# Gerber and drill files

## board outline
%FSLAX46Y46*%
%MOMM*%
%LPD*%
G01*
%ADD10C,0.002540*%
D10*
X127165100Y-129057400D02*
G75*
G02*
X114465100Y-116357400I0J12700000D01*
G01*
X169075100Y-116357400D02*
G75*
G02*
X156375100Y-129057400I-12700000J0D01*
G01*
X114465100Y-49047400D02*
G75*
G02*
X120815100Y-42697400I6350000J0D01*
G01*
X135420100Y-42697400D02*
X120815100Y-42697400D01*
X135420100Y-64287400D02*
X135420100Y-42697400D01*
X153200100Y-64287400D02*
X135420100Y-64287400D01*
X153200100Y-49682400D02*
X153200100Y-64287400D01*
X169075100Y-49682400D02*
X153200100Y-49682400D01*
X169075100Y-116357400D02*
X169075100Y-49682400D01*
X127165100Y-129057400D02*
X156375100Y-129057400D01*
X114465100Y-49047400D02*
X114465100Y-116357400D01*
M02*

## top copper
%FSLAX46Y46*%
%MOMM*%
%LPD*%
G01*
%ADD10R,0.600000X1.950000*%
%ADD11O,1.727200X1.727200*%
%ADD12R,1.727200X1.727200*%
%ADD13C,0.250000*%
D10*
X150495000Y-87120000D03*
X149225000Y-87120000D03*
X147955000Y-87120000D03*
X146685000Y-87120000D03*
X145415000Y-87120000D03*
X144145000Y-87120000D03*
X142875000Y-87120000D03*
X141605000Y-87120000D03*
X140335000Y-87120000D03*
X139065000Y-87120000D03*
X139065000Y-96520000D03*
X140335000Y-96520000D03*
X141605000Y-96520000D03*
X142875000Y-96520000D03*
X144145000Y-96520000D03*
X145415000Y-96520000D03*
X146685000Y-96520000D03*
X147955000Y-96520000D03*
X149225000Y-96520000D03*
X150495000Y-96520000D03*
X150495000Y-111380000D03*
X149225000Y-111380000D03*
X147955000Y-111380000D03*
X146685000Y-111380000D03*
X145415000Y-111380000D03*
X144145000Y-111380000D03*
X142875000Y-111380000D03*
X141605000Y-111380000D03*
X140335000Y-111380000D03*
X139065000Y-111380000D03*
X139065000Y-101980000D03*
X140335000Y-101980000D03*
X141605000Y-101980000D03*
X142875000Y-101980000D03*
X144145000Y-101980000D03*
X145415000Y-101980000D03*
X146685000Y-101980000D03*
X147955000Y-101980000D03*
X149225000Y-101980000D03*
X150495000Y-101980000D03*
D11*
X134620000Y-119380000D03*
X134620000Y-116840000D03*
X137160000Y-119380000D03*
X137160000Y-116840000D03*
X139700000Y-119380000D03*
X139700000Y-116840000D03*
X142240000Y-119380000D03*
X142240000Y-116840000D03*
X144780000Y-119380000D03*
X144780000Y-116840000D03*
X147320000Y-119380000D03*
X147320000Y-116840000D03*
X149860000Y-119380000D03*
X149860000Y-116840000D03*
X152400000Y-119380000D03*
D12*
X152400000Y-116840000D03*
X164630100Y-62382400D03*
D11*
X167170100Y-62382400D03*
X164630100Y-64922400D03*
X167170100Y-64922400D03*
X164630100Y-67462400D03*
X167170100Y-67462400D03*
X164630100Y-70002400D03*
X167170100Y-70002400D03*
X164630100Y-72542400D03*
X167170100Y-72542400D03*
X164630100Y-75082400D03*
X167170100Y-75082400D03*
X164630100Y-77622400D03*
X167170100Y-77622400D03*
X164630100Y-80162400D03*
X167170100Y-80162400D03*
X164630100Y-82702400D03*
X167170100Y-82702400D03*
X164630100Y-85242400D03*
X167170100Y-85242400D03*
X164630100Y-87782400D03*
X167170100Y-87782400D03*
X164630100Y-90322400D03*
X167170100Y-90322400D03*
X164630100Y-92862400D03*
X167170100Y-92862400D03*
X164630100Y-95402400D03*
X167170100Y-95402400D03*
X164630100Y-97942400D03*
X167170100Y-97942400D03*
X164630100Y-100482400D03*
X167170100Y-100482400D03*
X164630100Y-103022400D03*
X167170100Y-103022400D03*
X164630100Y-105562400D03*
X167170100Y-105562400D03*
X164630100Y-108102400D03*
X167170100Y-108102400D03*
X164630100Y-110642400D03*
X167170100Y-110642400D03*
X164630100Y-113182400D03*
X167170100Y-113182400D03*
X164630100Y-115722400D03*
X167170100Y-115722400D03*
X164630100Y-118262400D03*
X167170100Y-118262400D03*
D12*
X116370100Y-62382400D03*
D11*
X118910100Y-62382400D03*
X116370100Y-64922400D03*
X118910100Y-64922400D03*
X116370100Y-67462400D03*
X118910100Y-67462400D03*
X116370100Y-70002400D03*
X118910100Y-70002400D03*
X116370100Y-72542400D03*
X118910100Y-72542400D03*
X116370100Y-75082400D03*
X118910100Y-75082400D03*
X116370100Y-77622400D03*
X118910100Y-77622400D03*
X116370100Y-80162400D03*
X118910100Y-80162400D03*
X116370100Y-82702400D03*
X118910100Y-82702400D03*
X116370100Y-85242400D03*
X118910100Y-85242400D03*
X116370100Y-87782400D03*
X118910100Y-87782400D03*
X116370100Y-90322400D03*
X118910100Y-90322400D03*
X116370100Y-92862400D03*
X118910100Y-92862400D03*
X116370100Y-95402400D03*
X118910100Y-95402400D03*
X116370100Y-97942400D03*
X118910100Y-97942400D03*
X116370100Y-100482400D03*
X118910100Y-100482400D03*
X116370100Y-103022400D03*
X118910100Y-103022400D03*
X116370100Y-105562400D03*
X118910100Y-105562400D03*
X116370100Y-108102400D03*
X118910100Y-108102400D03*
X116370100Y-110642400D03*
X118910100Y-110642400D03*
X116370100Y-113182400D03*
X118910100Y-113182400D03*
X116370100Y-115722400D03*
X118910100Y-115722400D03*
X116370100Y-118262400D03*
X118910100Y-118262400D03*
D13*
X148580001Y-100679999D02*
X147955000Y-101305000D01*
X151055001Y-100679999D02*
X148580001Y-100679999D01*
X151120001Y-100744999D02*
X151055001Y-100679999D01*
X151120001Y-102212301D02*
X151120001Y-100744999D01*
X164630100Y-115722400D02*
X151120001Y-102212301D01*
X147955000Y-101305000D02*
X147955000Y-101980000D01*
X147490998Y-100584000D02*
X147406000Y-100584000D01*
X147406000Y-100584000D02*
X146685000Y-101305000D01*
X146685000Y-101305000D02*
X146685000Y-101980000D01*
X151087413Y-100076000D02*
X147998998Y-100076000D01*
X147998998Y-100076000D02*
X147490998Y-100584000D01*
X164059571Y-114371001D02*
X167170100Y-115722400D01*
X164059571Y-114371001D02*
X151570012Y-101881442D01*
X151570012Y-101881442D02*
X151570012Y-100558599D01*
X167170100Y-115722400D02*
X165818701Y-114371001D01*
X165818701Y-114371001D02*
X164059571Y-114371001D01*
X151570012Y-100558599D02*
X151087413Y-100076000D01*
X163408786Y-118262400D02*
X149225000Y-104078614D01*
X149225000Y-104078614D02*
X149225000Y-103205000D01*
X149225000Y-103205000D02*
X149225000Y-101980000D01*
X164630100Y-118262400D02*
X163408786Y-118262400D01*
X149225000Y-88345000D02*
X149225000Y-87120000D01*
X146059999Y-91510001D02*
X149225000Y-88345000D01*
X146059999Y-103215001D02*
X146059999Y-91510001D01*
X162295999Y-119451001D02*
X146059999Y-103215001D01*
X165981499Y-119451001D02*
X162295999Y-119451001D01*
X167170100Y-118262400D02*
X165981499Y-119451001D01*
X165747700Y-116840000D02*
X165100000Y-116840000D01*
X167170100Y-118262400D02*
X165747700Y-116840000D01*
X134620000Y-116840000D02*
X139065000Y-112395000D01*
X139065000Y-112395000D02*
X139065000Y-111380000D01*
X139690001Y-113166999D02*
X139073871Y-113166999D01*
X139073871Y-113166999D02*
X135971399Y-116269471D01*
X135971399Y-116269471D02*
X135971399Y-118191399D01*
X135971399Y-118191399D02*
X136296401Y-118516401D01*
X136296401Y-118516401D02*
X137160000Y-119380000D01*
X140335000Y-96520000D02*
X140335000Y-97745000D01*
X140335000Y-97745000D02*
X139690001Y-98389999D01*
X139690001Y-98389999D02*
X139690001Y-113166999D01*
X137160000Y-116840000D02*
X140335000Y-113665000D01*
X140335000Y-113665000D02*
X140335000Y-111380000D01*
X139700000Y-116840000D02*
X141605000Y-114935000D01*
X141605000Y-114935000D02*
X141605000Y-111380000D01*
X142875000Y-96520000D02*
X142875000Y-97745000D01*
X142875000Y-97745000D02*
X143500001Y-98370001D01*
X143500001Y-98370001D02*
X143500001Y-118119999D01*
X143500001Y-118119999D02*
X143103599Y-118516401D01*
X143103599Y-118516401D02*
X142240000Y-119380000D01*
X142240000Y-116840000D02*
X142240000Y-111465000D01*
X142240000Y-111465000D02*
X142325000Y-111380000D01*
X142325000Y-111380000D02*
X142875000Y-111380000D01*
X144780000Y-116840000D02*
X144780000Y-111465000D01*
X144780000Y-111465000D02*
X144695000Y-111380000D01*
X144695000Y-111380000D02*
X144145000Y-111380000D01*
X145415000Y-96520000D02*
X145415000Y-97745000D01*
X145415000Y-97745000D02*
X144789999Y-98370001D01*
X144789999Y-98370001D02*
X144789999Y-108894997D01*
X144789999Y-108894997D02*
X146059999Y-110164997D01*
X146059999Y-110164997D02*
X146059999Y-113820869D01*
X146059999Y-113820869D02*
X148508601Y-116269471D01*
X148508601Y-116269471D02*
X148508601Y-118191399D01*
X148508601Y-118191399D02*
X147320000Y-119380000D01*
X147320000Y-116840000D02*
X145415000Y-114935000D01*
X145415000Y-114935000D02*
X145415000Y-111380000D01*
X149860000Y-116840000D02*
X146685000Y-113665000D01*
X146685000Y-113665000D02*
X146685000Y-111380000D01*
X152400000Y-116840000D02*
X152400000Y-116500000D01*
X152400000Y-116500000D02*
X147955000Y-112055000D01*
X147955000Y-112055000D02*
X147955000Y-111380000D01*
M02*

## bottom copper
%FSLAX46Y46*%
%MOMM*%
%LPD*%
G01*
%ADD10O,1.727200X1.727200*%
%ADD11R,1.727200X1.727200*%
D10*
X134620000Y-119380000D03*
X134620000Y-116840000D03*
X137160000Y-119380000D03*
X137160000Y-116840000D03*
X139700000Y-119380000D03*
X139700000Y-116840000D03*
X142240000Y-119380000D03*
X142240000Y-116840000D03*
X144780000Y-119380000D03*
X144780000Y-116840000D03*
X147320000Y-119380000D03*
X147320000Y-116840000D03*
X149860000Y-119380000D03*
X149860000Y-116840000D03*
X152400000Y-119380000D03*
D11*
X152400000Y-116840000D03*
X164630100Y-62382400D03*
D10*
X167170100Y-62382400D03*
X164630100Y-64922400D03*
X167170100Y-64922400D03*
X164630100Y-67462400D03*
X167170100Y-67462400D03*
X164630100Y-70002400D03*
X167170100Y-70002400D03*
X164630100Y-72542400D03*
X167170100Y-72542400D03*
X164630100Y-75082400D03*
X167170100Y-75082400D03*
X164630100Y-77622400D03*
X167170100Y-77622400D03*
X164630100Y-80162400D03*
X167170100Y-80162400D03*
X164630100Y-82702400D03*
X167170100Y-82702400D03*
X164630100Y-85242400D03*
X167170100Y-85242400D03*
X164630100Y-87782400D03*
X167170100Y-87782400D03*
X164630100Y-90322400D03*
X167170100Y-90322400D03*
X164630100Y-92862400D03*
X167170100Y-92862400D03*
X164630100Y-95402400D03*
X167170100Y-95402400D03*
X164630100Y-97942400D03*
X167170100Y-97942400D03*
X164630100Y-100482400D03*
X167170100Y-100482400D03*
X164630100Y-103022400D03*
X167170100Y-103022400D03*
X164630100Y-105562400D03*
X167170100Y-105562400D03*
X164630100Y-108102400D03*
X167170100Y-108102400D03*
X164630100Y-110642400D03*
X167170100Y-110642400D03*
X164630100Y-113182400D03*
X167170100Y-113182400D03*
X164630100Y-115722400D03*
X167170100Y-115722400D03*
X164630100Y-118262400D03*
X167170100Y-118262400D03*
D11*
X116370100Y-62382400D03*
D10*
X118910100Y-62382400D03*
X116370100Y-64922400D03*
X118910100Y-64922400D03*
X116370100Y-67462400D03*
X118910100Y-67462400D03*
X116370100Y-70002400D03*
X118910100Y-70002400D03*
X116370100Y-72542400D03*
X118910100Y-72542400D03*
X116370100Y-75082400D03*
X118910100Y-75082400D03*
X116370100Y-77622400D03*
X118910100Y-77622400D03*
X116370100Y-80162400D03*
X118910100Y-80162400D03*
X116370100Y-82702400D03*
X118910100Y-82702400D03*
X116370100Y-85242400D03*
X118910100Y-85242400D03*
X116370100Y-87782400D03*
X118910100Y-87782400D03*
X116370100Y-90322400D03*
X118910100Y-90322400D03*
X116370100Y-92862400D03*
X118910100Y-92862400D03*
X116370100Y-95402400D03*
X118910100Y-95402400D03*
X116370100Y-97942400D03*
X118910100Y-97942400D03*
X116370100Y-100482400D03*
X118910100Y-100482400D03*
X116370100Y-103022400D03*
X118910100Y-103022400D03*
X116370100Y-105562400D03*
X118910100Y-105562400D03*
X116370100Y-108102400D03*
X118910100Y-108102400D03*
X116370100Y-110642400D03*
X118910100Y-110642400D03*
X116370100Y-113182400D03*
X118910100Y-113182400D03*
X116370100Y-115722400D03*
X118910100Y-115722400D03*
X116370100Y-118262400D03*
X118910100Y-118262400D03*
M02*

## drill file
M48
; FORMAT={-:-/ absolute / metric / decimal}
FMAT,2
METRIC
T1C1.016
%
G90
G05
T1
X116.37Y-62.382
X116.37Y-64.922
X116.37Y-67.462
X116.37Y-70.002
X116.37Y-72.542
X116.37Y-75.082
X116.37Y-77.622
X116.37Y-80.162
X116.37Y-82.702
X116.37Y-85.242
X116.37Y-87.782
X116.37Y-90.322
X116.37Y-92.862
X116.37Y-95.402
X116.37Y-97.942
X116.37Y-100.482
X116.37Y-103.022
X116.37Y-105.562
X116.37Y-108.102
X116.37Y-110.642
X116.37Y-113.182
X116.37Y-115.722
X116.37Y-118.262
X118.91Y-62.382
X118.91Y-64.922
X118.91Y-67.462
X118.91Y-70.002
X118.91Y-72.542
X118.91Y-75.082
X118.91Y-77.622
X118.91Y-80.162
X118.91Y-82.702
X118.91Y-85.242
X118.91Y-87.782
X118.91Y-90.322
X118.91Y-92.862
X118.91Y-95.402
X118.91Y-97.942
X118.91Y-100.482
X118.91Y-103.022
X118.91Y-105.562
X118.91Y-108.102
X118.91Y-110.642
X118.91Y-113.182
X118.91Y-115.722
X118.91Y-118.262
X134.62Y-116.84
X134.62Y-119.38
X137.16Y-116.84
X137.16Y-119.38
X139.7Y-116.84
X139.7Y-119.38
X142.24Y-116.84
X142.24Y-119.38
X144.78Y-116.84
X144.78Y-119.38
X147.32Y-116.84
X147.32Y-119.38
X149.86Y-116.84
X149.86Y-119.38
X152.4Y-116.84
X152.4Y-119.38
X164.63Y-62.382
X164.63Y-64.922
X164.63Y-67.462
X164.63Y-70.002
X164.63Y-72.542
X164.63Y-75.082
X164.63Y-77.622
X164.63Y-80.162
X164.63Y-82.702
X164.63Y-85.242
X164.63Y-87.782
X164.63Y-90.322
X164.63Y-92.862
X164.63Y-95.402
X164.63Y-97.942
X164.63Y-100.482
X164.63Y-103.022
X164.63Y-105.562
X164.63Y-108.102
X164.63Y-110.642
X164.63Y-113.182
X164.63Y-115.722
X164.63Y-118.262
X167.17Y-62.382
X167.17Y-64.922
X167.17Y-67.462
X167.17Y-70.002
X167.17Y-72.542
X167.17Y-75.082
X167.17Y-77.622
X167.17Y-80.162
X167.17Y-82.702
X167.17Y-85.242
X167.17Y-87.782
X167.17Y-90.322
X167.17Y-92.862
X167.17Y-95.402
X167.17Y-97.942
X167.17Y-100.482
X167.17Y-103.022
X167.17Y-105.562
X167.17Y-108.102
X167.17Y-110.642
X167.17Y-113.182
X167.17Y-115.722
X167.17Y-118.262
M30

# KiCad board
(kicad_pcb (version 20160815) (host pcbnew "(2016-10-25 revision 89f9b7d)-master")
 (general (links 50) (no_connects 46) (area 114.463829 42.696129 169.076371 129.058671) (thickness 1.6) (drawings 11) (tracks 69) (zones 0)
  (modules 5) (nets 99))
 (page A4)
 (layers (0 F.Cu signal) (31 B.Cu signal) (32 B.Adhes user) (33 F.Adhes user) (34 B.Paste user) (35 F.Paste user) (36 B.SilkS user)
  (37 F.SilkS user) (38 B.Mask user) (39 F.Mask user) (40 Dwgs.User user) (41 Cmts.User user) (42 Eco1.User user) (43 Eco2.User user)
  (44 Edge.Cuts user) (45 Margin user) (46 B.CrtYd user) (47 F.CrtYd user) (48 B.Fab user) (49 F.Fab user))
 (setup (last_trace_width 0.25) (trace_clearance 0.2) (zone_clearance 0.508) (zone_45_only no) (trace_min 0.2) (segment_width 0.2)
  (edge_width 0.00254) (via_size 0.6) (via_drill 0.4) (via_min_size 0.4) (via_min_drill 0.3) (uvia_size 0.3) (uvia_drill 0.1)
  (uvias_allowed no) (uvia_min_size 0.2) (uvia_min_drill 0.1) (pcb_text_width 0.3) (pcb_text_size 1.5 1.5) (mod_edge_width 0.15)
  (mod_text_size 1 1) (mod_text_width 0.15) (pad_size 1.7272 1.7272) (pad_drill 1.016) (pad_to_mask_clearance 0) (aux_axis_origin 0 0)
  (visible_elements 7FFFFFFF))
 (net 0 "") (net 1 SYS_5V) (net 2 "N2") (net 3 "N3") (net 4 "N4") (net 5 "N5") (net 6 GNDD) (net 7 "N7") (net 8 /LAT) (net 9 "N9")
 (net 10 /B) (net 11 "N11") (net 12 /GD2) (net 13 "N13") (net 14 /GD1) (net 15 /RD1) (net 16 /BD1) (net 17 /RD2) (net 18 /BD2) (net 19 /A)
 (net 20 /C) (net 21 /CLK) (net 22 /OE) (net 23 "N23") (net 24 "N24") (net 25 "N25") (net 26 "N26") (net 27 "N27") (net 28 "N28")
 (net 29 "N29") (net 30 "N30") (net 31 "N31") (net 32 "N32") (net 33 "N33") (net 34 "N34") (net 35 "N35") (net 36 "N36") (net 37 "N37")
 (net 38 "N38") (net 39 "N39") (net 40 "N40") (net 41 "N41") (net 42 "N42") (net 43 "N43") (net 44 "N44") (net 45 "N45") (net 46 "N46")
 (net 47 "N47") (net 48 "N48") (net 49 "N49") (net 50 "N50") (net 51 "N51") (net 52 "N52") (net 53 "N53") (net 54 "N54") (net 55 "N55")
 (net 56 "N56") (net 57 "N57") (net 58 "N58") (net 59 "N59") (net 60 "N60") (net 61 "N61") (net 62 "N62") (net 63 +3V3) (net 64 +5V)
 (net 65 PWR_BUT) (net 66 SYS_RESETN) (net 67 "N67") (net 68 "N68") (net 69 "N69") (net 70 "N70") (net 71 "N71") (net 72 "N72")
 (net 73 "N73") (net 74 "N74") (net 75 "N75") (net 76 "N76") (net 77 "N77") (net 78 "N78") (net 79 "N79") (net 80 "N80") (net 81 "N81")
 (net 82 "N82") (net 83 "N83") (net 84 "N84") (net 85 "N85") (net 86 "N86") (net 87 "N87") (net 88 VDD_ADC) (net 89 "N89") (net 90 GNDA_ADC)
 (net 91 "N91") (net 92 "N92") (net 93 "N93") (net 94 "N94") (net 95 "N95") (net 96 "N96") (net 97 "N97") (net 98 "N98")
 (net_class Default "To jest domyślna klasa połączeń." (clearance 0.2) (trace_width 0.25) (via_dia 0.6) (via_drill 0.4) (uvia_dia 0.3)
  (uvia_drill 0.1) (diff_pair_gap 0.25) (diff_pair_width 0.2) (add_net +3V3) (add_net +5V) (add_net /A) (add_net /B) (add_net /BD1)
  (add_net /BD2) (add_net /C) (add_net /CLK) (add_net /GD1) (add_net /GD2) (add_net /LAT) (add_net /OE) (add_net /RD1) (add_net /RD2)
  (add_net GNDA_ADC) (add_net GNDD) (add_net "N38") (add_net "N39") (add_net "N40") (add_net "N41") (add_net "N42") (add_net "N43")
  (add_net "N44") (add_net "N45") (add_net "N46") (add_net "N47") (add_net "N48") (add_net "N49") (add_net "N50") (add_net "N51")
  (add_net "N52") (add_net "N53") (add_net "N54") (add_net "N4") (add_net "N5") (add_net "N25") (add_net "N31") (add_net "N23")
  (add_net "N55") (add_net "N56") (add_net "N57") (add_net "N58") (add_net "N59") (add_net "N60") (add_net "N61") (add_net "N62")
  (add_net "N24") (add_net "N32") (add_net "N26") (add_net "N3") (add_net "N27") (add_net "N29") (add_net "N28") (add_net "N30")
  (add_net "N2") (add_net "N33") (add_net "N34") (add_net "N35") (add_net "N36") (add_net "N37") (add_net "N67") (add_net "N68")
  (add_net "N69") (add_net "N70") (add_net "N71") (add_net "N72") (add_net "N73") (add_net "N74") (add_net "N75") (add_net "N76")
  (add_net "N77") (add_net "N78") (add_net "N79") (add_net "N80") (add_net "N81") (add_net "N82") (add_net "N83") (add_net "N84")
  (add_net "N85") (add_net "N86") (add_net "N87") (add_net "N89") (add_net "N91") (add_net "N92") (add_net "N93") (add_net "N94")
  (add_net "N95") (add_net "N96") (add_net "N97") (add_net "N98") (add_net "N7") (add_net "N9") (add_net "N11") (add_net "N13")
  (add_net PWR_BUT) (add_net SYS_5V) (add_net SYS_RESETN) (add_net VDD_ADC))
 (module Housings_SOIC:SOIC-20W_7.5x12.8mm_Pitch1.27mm (layer F.Cu) (at 144.78 91.82 270)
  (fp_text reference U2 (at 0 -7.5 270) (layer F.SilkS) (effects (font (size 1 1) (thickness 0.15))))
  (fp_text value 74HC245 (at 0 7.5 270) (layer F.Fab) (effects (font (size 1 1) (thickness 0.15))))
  (pad 1 smd rect (at -4.7 -5.715 270) (size 1.95 0.6) (layers F.Cu F.Paste F.Mask) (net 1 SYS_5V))
  (pad 2 smd rect (at -4.7 -4.445 270) (size 1.95 0.6) (layers F.Cu F.Paste F.Mask) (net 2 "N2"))
  (pad 3 smd rect (at -4.7 -3.175 270) (size 1.95 0.6) (layers F.Cu F.Paste F.Mask) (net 1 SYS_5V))
  (pad 4 smd rect (at -4.7 -1.905 270) (size 1.95 0.6) (layers F.Cu F.Paste F.Mask) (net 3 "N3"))
  (pad 5 smd rect (at -4.7 -0.635 270) (size 1.95 0.6) (layers F.Cu F.Paste F.Mask) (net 1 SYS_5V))
  (pad 6 smd rect (at -4.7 0.635 270) (size 1.95 0.6) (layers F.Cu F.Paste F.Mask) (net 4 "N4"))
  (pad 7 smd rect (at -4.7 1.905 270) (size 1.95 0.6) (layers F.Cu F.Paste F.Mask) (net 1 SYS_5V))
  (pad 8 smd rect (at -4.7 3.175 270) (size 1.95 0.6) (layers F.Cu F.Paste F.Mask) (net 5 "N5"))
  (pad 9 smd rect (at -4.7 4.445 270) (size 1.95 0.6) (layers F.Cu F.Paste F.Mask) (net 1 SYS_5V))
  (pad 10 smd rect (at -4.7 5.715 270) (size 1.95 0.6) (layers F.Cu F.Paste F.Mask) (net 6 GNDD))
  (pad 11 smd rect (at 4.7 5.715 270) (size 1.95 0.6) (layers F.Cu F.Paste F.Mask) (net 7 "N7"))
  (pad 12 smd rect (at 4.7 4.445 270) (size 1.95 0.6) (layers F.Cu F.Paste F.Mask) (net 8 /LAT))
  (pad 13 smd rect (at 4.7 3.175 270) (size 1.95 0.6) (layers F.Cu F.Paste F.Mask) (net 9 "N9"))
  (pad 14 smd rect (at 4.7 1.905 270) (size 1.95 0.6) (layers F.Cu F.Paste F.Mask) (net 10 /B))
  (pad 15 smd rect (at 4.7 0.635 270) (size 1.95 0.6) (layers F.Cu F.Paste F.Mask) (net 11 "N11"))
  (pad 16 smd rect (at 4.7 -0.635 270) (size 1.95 0.6) (layers F.Cu F.Paste F.Mask) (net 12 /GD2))
  (pad 17 smd rect (at 4.7 -1.905 270) (size 1.95 0.6) (layers F.Cu F.Paste F.Mask) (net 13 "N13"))
  (pad 18 smd rect (at 4.7 -3.175 270) (size 1.95 0.6) (layers F.Cu F.Paste F.Mask) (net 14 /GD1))
  (pad 19 smd rect (at 4.7 -4.445 270) (size 1.95 0.6) (layers F.Cu F.Paste F.Mask) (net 6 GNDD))
  (pad 20 smd rect (at 4.7 -5.715 270) (size 1.95 0.6) (layers F.Cu F.Paste F.Mask) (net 1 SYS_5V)))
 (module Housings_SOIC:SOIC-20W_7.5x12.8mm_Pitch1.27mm (layer F.Cu) (at 144.78 106.68 270)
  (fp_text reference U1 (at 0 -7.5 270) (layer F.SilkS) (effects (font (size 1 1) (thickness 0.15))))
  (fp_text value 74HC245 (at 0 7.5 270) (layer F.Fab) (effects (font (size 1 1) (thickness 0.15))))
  (pad 20 smd rect (at 4.7 -5.715 270) (size 1.95 0.6) (layers F.Cu F.Paste F.Mask) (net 1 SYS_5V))
  (pad 19 smd rect (at 4.7 -4.445 270) (size 1.95 0.6) (layers F.Cu F.Paste F.Mask) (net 6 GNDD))
  (pad 18 smd rect (at 4.7 -3.175 270) (size 1.95 0.6) (layers F.Cu F.Paste F.Mask) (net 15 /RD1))
  (pad 17 smd rect (at 4.7 -1.905 270) (size 1.95 0.6) (layers F.Cu F.Paste F.Mask) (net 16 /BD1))
  (pad 16 smd rect (at 4.7 -0.635 270) (size 1.95 0.6) (layers F.Cu F.Paste F.Mask) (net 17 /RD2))
  (pad 15 smd rect (at 4.7 0.635 270) (size 1.95 0.6) (layers F.Cu F.Paste F.Mask) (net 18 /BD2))
  (pad 14 smd rect (at 4.7 1.905 270) (size 1.95 0.6) (layers F.Cu F.Paste F.Mask) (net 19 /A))
  (pad 13 smd rect (at 4.7 3.175 270) (size 1.95 0.6) (layers F.Cu F.Paste F.Mask) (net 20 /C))
  (pad 12 smd rect (at 4.7 4.445 270) (size 1.95 0.6) (layers F.Cu F.Paste F.Mask) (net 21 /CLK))
  (pad 11 smd rect (at 4.7 5.715 270) (size 1.95 0.6) (layers F.Cu F.Paste F.Mask) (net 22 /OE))
  (pad 10 smd rect (at -4.7 5.715 270) (size 1.95 0.6) (layers F.Cu F.Paste F.Mask) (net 6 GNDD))
  (pad 9 smd rect (at -4.7 4.445 270) (size 1.95 0.6) (layers F.Cu F.Paste F.Mask) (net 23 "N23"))
  (pad 8 smd rect (at -4.7 3.175 270) (size 1.95 0.6) (layers F.Cu F.Paste F.Mask) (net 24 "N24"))
  (pad 7 smd rect (at -4.7 1.905 270) (size 1.95 0.6) (layers F.Cu F.Paste F.Mask) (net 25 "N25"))
  (pad 6 smd rect (at -4.7 0.635 270) (size 1.95 0.6) (layers F.Cu F.Paste F.Mask) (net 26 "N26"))
  (pad 5 smd rect (at -4.7 -0.635 270) (size 1.95 0.6) (layers F.Cu F.Paste F.Mask) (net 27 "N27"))
  (pad 4 smd rect (at -4.7 -1.905 270) (size 1.95 0.6) (layers F.Cu F.Paste F.Mask) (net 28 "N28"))
  (pad 3 smd rect (at -4.7 -3.175 270) (size 1.95 0.6) (layers F.Cu F.Paste F.Mask) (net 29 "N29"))
  (pad 2 smd rect (at -4.7 -4.445 270) (size 1.95 0.6) (layers F.Cu F.Paste F.Mask) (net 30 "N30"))
  (pad 1 smd rect (at -4.7 -5.715 270) (size 1.95 0.6) (layers F.Cu F.Paste F.Mask) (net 1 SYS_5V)))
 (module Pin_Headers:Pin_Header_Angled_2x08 (layer F.Cu) (at 152.4 116.84 270)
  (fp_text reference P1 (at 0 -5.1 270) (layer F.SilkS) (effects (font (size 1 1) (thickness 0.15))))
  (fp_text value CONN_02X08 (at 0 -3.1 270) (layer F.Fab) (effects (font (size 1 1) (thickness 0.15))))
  (pad 16 thru_hole oval (at 2.54 17.78 270) (size 1.7272 1.7272) (drill 1.016) (layers *.Cu *.Mask F.SilkS) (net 6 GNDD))
  (pad 15 thru_hole oval (at 0 17.78 270) (size 1.7272 1.7272) (drill 1.016) (layers *.Cu *.Mask F.SilkS) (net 22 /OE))
  (pad 14 thru_hole oval (at 2.54 15.24 270) (size 1.7272 1.7272) (drill 1.016) (layers *.Cu *.Mask F.SilkS) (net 8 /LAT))
  (pad 13 thru_hole oval (at 0 15.24 270) (size 1.7272 1.7272) (drill 1.016) (layers *.Cu *.Mask F.SilkS) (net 21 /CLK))
  (pad 12 thru_hole oval (at 2.54 12.7 270) (size 1.7272 1.7272) (drill 1.016) (layers *.Cu *.Mask F.SilkS) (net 6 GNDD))
  (pad 11 thru_hole oval (at 0 12.7 270) (size 1.7272 1.7272) (drill 1.016) (layers *.Cu *.Mask F.SilkS) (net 20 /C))
  (pad 10 thru_hole oval (at 2.54 10.16 270) (size 1.7272 1.7272) (drill 1.016) (layers *.Cu *.Mask F.SilkS) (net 10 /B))
  (pad 9 thru_hole oval (at 0 10.16 270) (size 1.7272 1.7272) (drill 1.016) (layers *.Cu *.Mask F.SilkS) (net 19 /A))
  (pad 8 thru_hole oval (at 2.54 7.62 270) (size 1.7272 1.7272) (drill 1.016) (layers *.Cu *.Mask F.SilkS) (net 6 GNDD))
  (pad 7 thru_hole oval (at 0 7.62 270) (size 1.7272 1.7272) (drill 1.016) (layers *.Cu *.Mask F.SilkS) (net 18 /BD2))
  (pad 6 thru_hole oval (at 2.54 5.08 270) (size 1.7272 1.7272) (drill 1.016) (layers *.Cu *.Mask F.SilkS) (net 12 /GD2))
  (pad 5 thru_hole oval (at 0 5.08 270) (size 1.7272 1.7272) (drill 1.016) (layers *.Cu *.Mask F.SilkS) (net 17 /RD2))
  (pad 4 thru_hole oval (at 2.54 2.54 270) (size 1.7272 1.7272) (drill 1.016) (layers *.Cu *.Mask F.SilkS) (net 6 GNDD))
  (pad 3 thru_hole oval (at 0 2.54 270) (size 1.7272 1.7272) (drill 1.016) (layers *.Cu *.Mask F.SilkS) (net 16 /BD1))
  (pad 2 thru_hole oval (at 2.54 0 270) (size 1.7272 1.7272) (drill 1.016) (layers *.Cu *.Mask F.SilkS) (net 14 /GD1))
  (pad 1 thru_hole rect (at 0 0 270) (size 1.7272 1.7272) (drill 1.016) (layers *.Cu *.Mask F.SilkS) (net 15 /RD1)))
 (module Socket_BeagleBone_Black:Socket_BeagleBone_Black (layer F.Cu) (at 164.6301 62.3824)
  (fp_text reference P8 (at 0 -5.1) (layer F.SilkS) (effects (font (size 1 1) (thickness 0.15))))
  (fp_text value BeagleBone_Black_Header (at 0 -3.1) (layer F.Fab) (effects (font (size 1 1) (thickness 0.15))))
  (pad 1 thru_hole rect (at 0 0) (size 1.7272 1.7272) (drill 1.016) (layers *.Cu *.Mask F.SilkS) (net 6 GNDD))
  (pad 2 thru_hole oval (at 2.54 0) (size 1.7272 1.7272) (drill 1.016) (layers *.Cu *.Mask F.SilkS) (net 6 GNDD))
  (pad 3 thru_hole oval (at 0 2.54) (size 1.7272 1.7272) (drill 1.016) (layers *.Cu *.Mask F.SilkS) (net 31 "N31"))
  (pad 4 thru_hole oval (at 2.54 2.54) (size 1.7272 1.7272) (drill 1.016) (layers *.Cu *.Mask F.SilkS) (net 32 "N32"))
  (pad 5 thru_hole oval (at 0 5.08) (size 1.7272 1.7272) (drill 1.016) (layers *.Cu *.Mask F.SilkS) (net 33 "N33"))
  (pad 6 thru_hole oval (at 2.54 5.08) (size 1.7272 1.7272) (drill 1.016) (layers *.Cu *.Mask F.SilkS) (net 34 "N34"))
  (pad 7 thru_hole oval (at 0 7.62) (size 1.7272 1.7272) (drill 1.016) (layers *.Cu *.Mask F.SilkS) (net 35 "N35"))
  (pad 8 thru_hole oval (at 2.54 7.62) (size 1.7272 1.7272) (drill 1.016) (layers *.Cu *.Mask F.SilkS) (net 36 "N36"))
  (pad 9 thru_hole oval (at 0 10.16) (size 1.7272 1.7272) (drill 1.016) (layers *.Cu *.Mask F.SilkS) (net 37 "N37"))
  (pad 10 thru_hole oval (at 2.54 10.16) (size 1.7272 1.7272) (drill 1.016) (layers *.Cu *.Mask F.SilkS) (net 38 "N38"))
  (pad 11 thru_hole oval (at 0 12.7) (size 1.7272 1.7272) (drill 1.016) (layers *.Cu *.Mask F.SilkS) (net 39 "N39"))
  (pad 12 thru_hole oval (at 2.54 12.7) (size 1.7272 1.7272) (drill 1.016) (layers *.Cu *.Mask F.SilkS) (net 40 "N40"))
  (pad 13 thru_hole oval (at 0 15.24) (size 1.7272 1.7272) (drill 1.016) (layers *.Cu *.Mask F.SilkS) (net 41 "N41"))
  (pad 14 thru_hole oval (at 2.54 15.24) (size 1.7272 1.7272) (drill 1.016) (layers *.Cu *.Mask F.SilkS) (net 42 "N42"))
  (pad 15 thru_hole oval (at 0 17.78) (size 1.7272 1.7272) (drill 1.016) (layers *.Cu *.Mask F.SilkS) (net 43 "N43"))
  (pad 16 thru_hole oval (at 2.54 17.78) (size 1.7272 1.7272) (drill 1.016) (layers *.Cu *.Mask F.SilkS) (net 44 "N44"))
  (pad 17 thru_hole oval (at 0 20.32) (size 1.7272 1.7272) (drill 1.016) (layers *.Cu *.Mask F.SilkS) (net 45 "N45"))
  (pad 18 thru_hole oval (at 2.54 20.32) (size 1.7272 1.7272) (drill 1.016) (layers *.Cu *.Mask F.SilkS) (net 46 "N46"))
  (pad 19 thru_hole oval (at 0 22.86) (size 1.7272 1.7272) (drill 1.016) (layers *.Cu *.Mask F.SilkS) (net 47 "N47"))
  (pad 20 thru_hole oval (at 2.54 22.86) (size 1.7272 1.7272) (drill 1.016) (layers *.Cu *.Mask F.SilkS) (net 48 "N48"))
  (pad 21 thru_hole oval (at 0 25.4) (size 1.7272 1.7272) (drill 1.016) (layers *.Cu *.Mask F.SilkS) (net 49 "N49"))
  (pad 22 thru_hole oval (at 2.54 25.4) (size 1.7272 1.7272) (drill 1.016) (layers *.Cu *.Mask F.SilkS) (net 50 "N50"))
  (pad 23 thru_hole oval (at 0 27.94) (size 1.7272 1.7272) (drill 1.016) (layers *.Cu *.Mask F.SilkS) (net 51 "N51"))
  (pad 24 thru_hole oval (at 2.54 27.94) (size 1.7272 1.7272) (drill 1.016) (layers *.Cu *.Mask F.SilkS) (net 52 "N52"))
  (pad 25 thru_hole oval (at 0 30.48) (size 1.7272 1.7272) (drill 1.016) (layers *.Cu *.Mask F.SilkS) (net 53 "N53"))
  (pad 26 thru_hole oval (at 2.54 30.48) (size 1.7272 1.7272) (drill 1.016) (layers *.Cu *.Mask F.SilkS) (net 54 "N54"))
  (pad 27 thru_hole oval (at 0 33.02) (size 1.7272 1.7272) (drill 1.016) (layers *.Cu *.Mask F.SilkS) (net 4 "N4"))
  (pad 28 thru_hole oval (at 2.54 33.02) (size 1.7272 1.7272) (drill 1.016) (layers *.Cu *.Mask F.SilkS) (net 5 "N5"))
  (pad 29 thru_hole oval (at 0 35.56) (size 1.7272 1.7272) (drill 1.016) (layers *.Cu *.Mask F.SilkS) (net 25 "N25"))
  (pad 30 thru_hole oval (at 2.54 35.56) (size 1.7272 1.7272) (drill 1.016) (layers *.Cu *.Mask F.SilkS) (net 23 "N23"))
  (pad 31 thru_hole oval (at 0 38.1) (size 1.7272 1.7272) (drill 1.016) (layers *.Cu *.Mask F.SilkS) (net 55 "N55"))
  (pad 32 thru_hole oval (at 2.54 38.1) (size 1.7272 1.7272) (drill 1.016) (layers *.Cu *.Mask F.SilkS) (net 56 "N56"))
  (pad 33 thru_hole oval (at 0 40.64) (size 1.7272 1.7272) (drill 1.016) (layers *.Cu *.Mask F.SilkS) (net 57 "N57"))
  (pad 34 thru_hole oval (at 2.54 40.64) (size 1.7272 1.7272) (drill 1.016) (layers *.Cu *.Mask F.SilkS) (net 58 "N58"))
  (pad 35 thru_hole oval (at 0 43.18) (size 1.7272 1.7272) (drill 1.016) (layers *.Cu *.Mask F.SilkS) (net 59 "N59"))
  (pad 36 thru_hole oval (at 2.54 43.18) (size 1.7272 1.7272) (drill 1.016) (layers *.Cu *.Mask F.SilkS) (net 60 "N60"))
  (pad 37 thru_hole oval (at 0 45.72) (size 1.7272 1.7272) (drill 1.016) (layers *.Cu *.Mask F.SilkS) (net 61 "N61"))
  (pad 38 thru_hole oval (at 2.54 45.72) (size 1.7272 1.7272) (drill 1.016) (layers *.Cu *.Mask F.SilkS) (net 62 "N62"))
  (pad 39 thru_hole oval (at 0 48.26) (size 1.7272 1.7272) (drill 1.016) (layers *.Cu *.Mask F.SilkS) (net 24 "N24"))
  (pad 40 thru_hole oval (at 2.54 48.26) (size 1.7272 1.7272) (drill 1.016) (layers *.Cu *.Mask F.SilkS) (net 26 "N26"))
  (pad 41 thru_hole oval (at 0 50.8) (size 1.7272 1.7272) (drill 1.016) (layers *.Cu *.Mask F.SilkS) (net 3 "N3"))
  (pad 42 thru_hole oval (at 2.54 50.8) (size 1.7272 1.7272) (drill 1.016) (layers *.Cu *.Mask F.SilkS) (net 27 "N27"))
  (pad 43 thru_hole oval (at 0 53.34) (size 1.7272 1.7272) (drill 1.016) (layers *.Cu *.Mask F.SilkS) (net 29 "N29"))
  (pad 44 thru_hole oval (at 2.54 53.34) (size 1.7272 1.7272) (drill 1.016) (layers *.Cu *.Mask F.SilkS) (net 28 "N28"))
  (pad 45 thru_hole oval (at 0 55.88) (size 1.7272 1.7272) (drill 1.016) (layers *.Cu *.Mask F.SilkS) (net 30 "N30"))
  (pad 46 thru_hole oval (at 2.54 55.88) (size 1.7272 1.7272) (drill 1.016) (layers *.Cu *.Mask F.SilkS) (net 2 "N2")))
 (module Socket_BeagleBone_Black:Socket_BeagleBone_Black (layer F.Cu) (at 116.3701 62.3824)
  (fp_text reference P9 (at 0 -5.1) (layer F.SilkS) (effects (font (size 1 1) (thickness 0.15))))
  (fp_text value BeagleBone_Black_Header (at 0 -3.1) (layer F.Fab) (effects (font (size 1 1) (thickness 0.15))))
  (pad 1 thru_hole rect (at 0 0) (size 1.7272 1.7272) (drill 1.016) (layers *.Cu *.Mask F.SilkS) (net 6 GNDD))
  (pad 2 thru_hole oval (at 2.54 0) (size 1.7272 1.7272) (drill 1.016) (layers *.Cu *.Mask F.SilkS) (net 6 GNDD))
  (pad 3 thru_hole oval (at 0 2.54) (size 1.7272 1.7272) (drill 1.016) (layers *.Cu *.Mask F.SilkS) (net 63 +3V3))
  (pad 4 thru_hole oval (at 2.54 2.54) (size 1.7272 1.7272) (drill 1.016) (layers *.Cu *.Mask F.SilkS) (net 63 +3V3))
  (pad 5 thru_hole oval (at 0 5.08) (size 1.7272 1.7272) (drill 1.016) (layers *.Cu *.Mask F.SilkS) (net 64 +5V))
  (pad 6 thru_hole oval (at 2.54 5.08) (size 1.7272 1.7272) (drill 1.016) (layers *.Cu *.Mask F.SilkS) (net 64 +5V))
  (pad 7 thru_hole oval (at 0 7.62) (size 1.7272 1.7272) (drill 1.016) (layers *.Cu *.Mask F.SilkS) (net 1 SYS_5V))
  (pad 8 thru_hole oval (at 2.54 7.62) (size 1.7272 1.7272) (drill 1.016) (layers *.Cu *.Mask F.SilkS) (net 1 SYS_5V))
  (pad 9 thru_hole oval (at 0 10.16) (size 1.7272 1.7272) (drill 1.016) (layers *.Cu *.Mask F.SilkS) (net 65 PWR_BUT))
  (pad 10 thru_hole oval (at 2.54 10.16) (size 1.7272 1.7272) (drill 1.016) (layers *.Cu *.Mask F.SilkS) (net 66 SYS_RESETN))
  (pad 11 thru_hole oval (at 0 12.7) (size 1.7272 1.7272) (drill 1.016) (layers *.Cu *.Mask F.SilkS) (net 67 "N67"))
  (pad 12 thru_hole oval (at 2.54 12.7) (size 1.7272 1.7272) (drill 1.016) (layers *.Cu *.Mask F.SilkS) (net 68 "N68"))
  (pad 13 thru_hole oval (at 0 15.24) (size 1.7272 1.7272) (drill 1.016) (layers *.Cu *.Mask F.SilkS) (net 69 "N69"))
  (pad 14 thru_hole oval (at 2.54 15.24) (size 1.7272 1.7272) (drill 1.016) (layers *.Cu *.Mask F.SilkS) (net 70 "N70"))
  (pad 15 thru_hole oval (at 0 17.78) (size 1.7272 1.7272) (drill 1.016) (layers *.Cu *.Mask F.SilkS) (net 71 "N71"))
  (pad 16 thru_hole oval (at 2.54 17.78) (size 1.7272 1.7272) (drill 1.016) (layers *.Cu *.Mask F.SilkS) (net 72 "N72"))
  (pad 17 thru_hole oval (at 0 20.32) (size 1.7272 1.7272) (drill 1.016) (layers *.Cu *.Mask F.SilkS) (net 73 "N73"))
  (pad 18 thru_hole oval (at 2.54 20.32) (size 1.7272 1.7272) (drill 1.016) (layers *.Cu *.Mask F.SilkS) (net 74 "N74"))
  (pad 19 thru_hole oval (at 0 22.86) (size 1.7272 1.7272) (drill 1.016) (layers *.Cu *.Mask F.SilkS) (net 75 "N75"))
  (pad 20 thru_hole oval (at 2.54 22.86) (size 1.7272 1.7272) (drill 1.016) (layers *.Cu *.Mask F.SilkS) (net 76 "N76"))
  (pad 21 thru_hole oval (at 0 25.4) (size 1.7272 1.7272) (drill 1.016) (layers *.Cu *.Mask F.SilkS) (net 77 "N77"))
  (pad 22 thru_hole oval (at 2.54 25.4) (size 1.7272 1.7272) (drill 1.016) (layers *.Cu *.Mask F.SilkS) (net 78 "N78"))
  (pad 23 thru_hole oval (at 0 27.94) (size 1.7272 1.7272) (drill 1.016) (layers *.Cu *.Mask F.SilkS) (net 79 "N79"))
  (pad 24 thru_hole oval (at 2.54 27.94) (size 1.7272 1.7272) (drill 1.016) (layers *.Cu *.Mask F.SilkS) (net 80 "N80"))
  (pad 25 thru_hole oval (at 0 30.48) (size 1.7272 1.7272) (drill 1.016) (layers *.Cu *.Mask F.SilkS) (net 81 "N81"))
  (pad 26 thru_hole oval (at 2.54 30.48) (size 1.7272 1.7272) (drill 1.016) (layers *.Cu *.Mask F.SilkS) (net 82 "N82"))
  (pad 27 thru_hole oval (at 0 33.02) (size 1.7272 1.7272) (drill 1.016) (layers *.Cu *.Mask F.SilkS) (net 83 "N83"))
  (pad 28 thru_hole oval (at 2.54 33.02) (size 1.7272 1.7272) (drill 1.016) (layers *.Cu *.Mask F.SilkS) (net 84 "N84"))
  (pad 29 thru_hole oval (at 0 35.56) (size 1.7272 1.7272) (drill 1.016) (layers *.Cu *.Mask F.SilkS) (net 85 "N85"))
  (pad 30 thru_hole oval (at 2.54 35.56) (size 1.7272 1.7272) (drill 1.016) (layers *.Cu *.Mask F.SilkS) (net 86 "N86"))
  (pad 31 thru_hole oval (at 0 38.1) (size 1.7272 1.7272) (drill 1.016) (layers *.Cu *.Mask F.SilkS) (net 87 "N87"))
  (pad 32 thru_hole oval (at 2.54 38.1) (size 1.7272 1.7272) (drill 1.016) (layers *.Cu *.Mask F.SilkS) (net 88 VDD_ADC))
  (pad 33 thru_hole oval (at 0 40.64) (size 1.7272 1.7272) (drill 1.016) (layers *.Cu *.Mask F.SilkS) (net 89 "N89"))
  (pad 34 thru_hole oval (at 2.54 40.64) (size 1.7272 1.7272) (drill 1.016) (layers *.Cu *.Mask F.SilkS) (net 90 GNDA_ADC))
  (pad 35 thru_hole oval (at 0 43.18) (size 1.7272 1.7272) (drill 1.016) (layers *.Cu *.Mask F.SilkS) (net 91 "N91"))
  (pad 36 thru_hole oval (at 2.54 43.18) (size 1.7272 1.7272) (drill 1.016) (layers *.Cu *.Mask F.SilkS) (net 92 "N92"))
  (pad 37 thru_hole oval (at 0 45.72) (size 1.7272 1.7272) (drill 1.016) (layers *.Cu *.Mask F.SilkS) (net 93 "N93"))
  (pad 38 thru_hole oval (at 2.54 45.72) (size 1.7272 1.7272) (drill 1.016) (layers *.Cu *.Mask F.SilkS) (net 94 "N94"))
  (pad 39 thru_hole oval (at 0 48.26) (size 1.7272 1.7272) (drill 1.016) (layers *.Cu *.Mask F.SilkS) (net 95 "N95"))
  (pad 40 thru_hole oval (at 2.54 48.26) (size 1.7272 1.7272) (drill 1.016) (layers *.Cu *.Mask F.SilkS) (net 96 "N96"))
  (pad 41 thru_hole oval (at 0 50.8) (size 1.7272 1.7272) (drill 1.016) (layers *.Cu *.Mask F.SilkS) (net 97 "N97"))
  (pad 42 thru_hole oval (at 2.54 50.8) (size 1.7272 1.7272) (drill 1.016) (layers *.Cu *.Mask F.SilkS) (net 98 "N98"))
  (pad 43 thru_hole oval (at 0 53.34) (size 1.7272 1.7272) (drill 1.016) (layers *.Cu *.Mask F.SilkS) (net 6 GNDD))
  (pad 44 thru_hole oval (at 2.54 53.34) (size 1.7272 1.7272) (drill 1.016) (layers *.Cu *.Mask F.SilkS) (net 6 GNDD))
  (pad 45 thru_hole oval (at 0 55.88) (size 1.7272 1.7272) (drill 1.016) (layers *.Cu *.Mask F.SilkS) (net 6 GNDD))
  (pad 46 thru_hole oval (at 2.54 55.88) (size 1.7272 1.7272) (drill 1.016) (layers *.Cu *.Mask F.SilkS) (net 6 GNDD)))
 (gr_arc (start 127.1651 116.3574) (end 127.1651 129.0574) (angle 90) (layer Edge.Cuts) (width 0.00254))
 (gr_arc (start 156.3751 116.3574) (end 169.0751 116.3574) (angle 90) (layer Edge.Cuts) (width 0.00254))
 (gr_arc (start 120.8151 49.0474) (end 114.4651 49.0474) (angle 90) (layer Edge.Cuts) (width 0.00254))
 (gr_line (start 135.4201 42.6974) (end 120.8151 42.6974) (layer Edge.Cuts) (width 0.00254))
 (gr_line (start 135.4201 64.2874) (end 135.4201 42.6974) (layer Edge.Cuts) (width 0.00254))
 (gr_line (start 153.2001 64.2874) (end 135.4201 64.2874) (layer Edge.Cuts) (width 0.00254))
 (gr_line (start 153.2001 49.6824) (end 153.2001 64.2874) (layer Edge.Cuts) (width 0.00254))
 (gr_line (start 169.0751 49.6824) (end 153.2001 49.6824) (layer Edge.Cuts) (width 0.00254))
 (gr_line (start 169.0751 116.3574) (end 169.0751 49.6824) (layer Edge.Cuts) (width 0.00254))
 (gr_line (start 127.1651 129.0574) (end 156.3751 129.0574) (layer Edge.Cuts) (width 0.00254))
 (gr_line (start 114.4651 49.0474) (end 114.4651 116.3574) (layer Edge.Cuts) (width 0.00254))
 (segment (start 148.580001 100.679999) (end 147.955 101.305) (width 0.25) (layer F.Cu) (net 29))
 (segment (start 151.055001 100.679999) (end 148.580001 100.679999) (width 0.25) (layer F.Cu) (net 29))
 (segment (start 151.120001 100.744999) (end 151.055001 100.679999) (width 0.25) (layer F.Cu) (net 29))
 (segment (start 151.120001 102.212301) (end 151.120001 100.744999) (width 0.25) (layer F.Cu) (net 29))
 (segment (start 164.6301 115.7224) (end 151.120001 102.212301) (width 0.25) (layer F.Cu) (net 29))
 (segment (start 147.955 101.305) (end 147.955 101.98) (width 0.25) (layer F.Cu) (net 29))
 (segment (start 147.490998 100.584) (end 147.406 100.584) (width 0.25) (layer F.Cu) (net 28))
 (segment (start 147.406 100.584) (end 146.685 101.305) (width 0.25) (layer F.Cu) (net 28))
 (segment (start 146.685 101.305) (end 146.685 101.98) (width 0.25) (layer F.Cu) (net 28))
 (segment (start 151.087413 100.076) (end 147.998998 100.076) (width 0.25) (layer F.Cu) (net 28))
 (segment (start 147.998998 100.076) (end 147.490998 100.584) (width 0.25) (layer F.Cu) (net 28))
 (segment (start 164.059571 114.371001) (end 167.1701 115.7224) (width 0.25) (layer F.Cu) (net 28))
 (segment (start 164.059571 114.371001) (end 151.570012 101.881442) (width 0.25) (layer F.Cu) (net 28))
 (segment (start 151.570012 101.881442) (end 151.570012 100.558599) (width 0.25) (layer F.Cu) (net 28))
 (segment (start 167.1701 115.7224) (end 165.818701 114.371001) (width 0.25) (layer F.Cu) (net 28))
 (segment (start 165.818701 114.371001) (end 164.059571 114.371001) (width 0.25) (layer F.Cu) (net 28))
 (segment (start 151.570012 100.558599) (end 151.087413 100.076) (width 0.25) (layer F.Cu) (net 28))
 (segment (start 163.408786 118.2624) (end 149.225 104.078614) (width 0.25) (layer F.Cu) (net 30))
 (segment (start 149.225 104.078614) (end 149.225 103.205) (width 0.25) (layer F.Cu) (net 30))
 (segment (start 149.225 103.205) (end 149.225 101.98) (width 0.25) (layer F.Cu) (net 30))
 (segment (start 164.6301 118.2624) (end 163.408786 118.2624) (width 0.25) (layer F.Cu) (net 30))
 (segment (start 149.225 88.345) (end 149.225 87.12) (width 0.25) (layer F.Cu) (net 2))
 (segment (start 146.059999 91.510001) (end 149.225 88.345) (width 0.25) (layer F.Cu) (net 2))
 (segment (start 146.059999 103.215001) (end 146.059999 91.510001) (width 0.25) (layer F.Cu) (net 2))
 (segment (start 162.295999 119.451001) (end 146.059999 103.215001) (width 0.25) (layer F.Cu) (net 2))
 (segment (start 165.981499 119.451001) (end 162.295999 119.451001) (width 0.25) (layer F.Cu) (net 2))
 (segment (start 167.1701 118.2624) (end 165.981499 119.451001) (width 0.25) (layer F.Cu) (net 2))
 (segment (start 165.7477 116.84) (end 165.1 116.84) (width 0.25) (layer F.Cu) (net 2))
 (segment (start 167.1701 118.2624) (end 165.7477 116.84) (width 0.25) (layer F.Cu) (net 2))
 (segment (start 134.62 116.84) (end 139.065 112.395) (width 0.25) (layer F.Cu) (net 22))
 (segment (start 139.065 112.395) (end 139.065 111.38) (width 0.25) (layer F.Cu) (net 22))
 (segment (start 139.690001 113.166999) (end 139.073871 113.166999) (width 0.25) (layer F.Cu) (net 8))
 (segment (start 139.073871 113.166999) (end 135.971399 116.269471) (width 0.25) (layer F.Cu) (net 8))
 (segment (start 135.971399 116.269471) (end 135.971399 118.191399) (width 0.25) (layer F.Cu) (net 8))
 (segment (start 135.971399 118.191399) (end 136.296401 118.516401) (width 0.25) (layer F.Cu) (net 8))
 (segment (start 136.296401 118.516401) (end 137.16 119.38) (width 0.25) (layer F.Cu) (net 8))
 (segment (start 140.335 96.52) (end 140.335 97.745) (width 0.25) (layer F.Cu) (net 8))
 (segment (start 140.335 97.745) (end 139.690001 98.389999) (width 0.25) (layer F.Cu) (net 8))
 (segment (start 139.690001 98.389999) (end 139.690001 113.166999) (width 0.25) (layer F.Cu) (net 8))
 (segment (start 137.16 116.84) (end 140.335 113.665) (width 0.25) (layer F.Cu) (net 21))
 (segment (start 140.335 113.665) (end 140.335 111.38) (width 0.25) (layer F.Cu) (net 21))
 (segment (start 139.7 116.84) (end 141.605 114.935) (width 0.25) (layer F.Cu) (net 20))
 (segment (start 141.605 114.935) (end 141.605 111.38) (width 0.25) (layer F.Cu) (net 20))
 (segment (start 142.875 96.52) (end 142.875 97.745) (width 0.25) (layer F.Cu) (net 10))
 (segment (start 142.875 97.745) (end 143.500001 98.370001) (width 0.25) (layer F.Cu) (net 10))
 (segment (start 143.500001 98.370001) (end 143.500001 118.119999) (width 0.25) (layer F.Cu) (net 10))
 (segment (start 143.500001 118.119999) (end 143.103599 118.516401) (width 0.25) (layer F.Cu) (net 10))
 (segment (start 143.103599 118.516401) (end 142.24 119.38) (width 0.25) (layer F.Cu) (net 10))
 (segment (start 142.24 116.84) (end 142.24 111.465) (width 0.25) (layer F.Cu) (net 19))
 (segment (start 142.24 111.465) (end 142.325 111.38) (width 0.25) (layer F.Cu) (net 19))
 (segment (start 142.325 111.38) (end 142.875 111.38) (width 0.25) (layer F.Cu) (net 19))
 (segment (start 144.78 116.84) (end 144.78 111.465) (width 0.25) (layer F.Cu) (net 18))
 (segment (start 144.78 111.465) (end 144.695 111.38) (width 0.25) (layer F.Cu) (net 18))
 (segment (start 144.695 111.38) (end 144.145 111.38) (width 0.25) (layer F.Cu) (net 18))
 (segment (start 145.415 96.52) (end 145.415 97.745) (width 0.25) (layer F.Cu) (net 12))
 (segment (start 145.415 97.745) (end 144.789999 98.370001) (width 0.25) (layer F.Cu) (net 12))
 (segment (start 144.789999 98.370001) (end 144.789999 108.894997) (width 0.25) (layer F.Cu) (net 12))
 (segment (start 144.789999 108.894997) (end 146.059999 110.164997) (width 0.25) (layer F.Cu) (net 12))
 (segment (start 146.059999 110.164997) (end 146.059999 113.820869) (width 0.25) (layer F.Cu) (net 12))
 (segment (start 146.059999 113.820869) (end 148.508601 116.269471) (width 0.25) (layer F.Cu) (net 12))
 (segment (start 148.508601 116.269471) (end 148.508601 118.191399) (width 0.25) (layer F.Cu) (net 12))
 (segment (start 148.508601 118.191399) (end 147.32 119.38) (width 0.25) (layer F.Cu) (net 12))
 (segment (start 147.32 116.84) (end 145.415 114.935) (width 0.25) (layer F.Cu) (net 17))
 (segment (start 145.415 114.935) (end 145.415 111.38) (width 0.25) (layer F.Cu) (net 17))
 (segment (start 149.86 116.84) (end 146.685 113.665) (width 0.25) (layer F.Cu) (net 16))
 (segment (start 146.685 113.665) (end 146.685 111.38) (width 0.25) (layer F.Cu) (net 16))
 (segment (start 152.4 116.84) (end 152.4 116.5) (width 0.25) (layer F.Cu) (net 15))
 (segment (start 152.4 116.5) (end 147.955 112.055) (width 0.25) (layer F.Cu) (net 15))
 (segment (start 147.955 112.055) (end 147.955 111.38) (width 0.25) (layer F.Cu) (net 15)))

